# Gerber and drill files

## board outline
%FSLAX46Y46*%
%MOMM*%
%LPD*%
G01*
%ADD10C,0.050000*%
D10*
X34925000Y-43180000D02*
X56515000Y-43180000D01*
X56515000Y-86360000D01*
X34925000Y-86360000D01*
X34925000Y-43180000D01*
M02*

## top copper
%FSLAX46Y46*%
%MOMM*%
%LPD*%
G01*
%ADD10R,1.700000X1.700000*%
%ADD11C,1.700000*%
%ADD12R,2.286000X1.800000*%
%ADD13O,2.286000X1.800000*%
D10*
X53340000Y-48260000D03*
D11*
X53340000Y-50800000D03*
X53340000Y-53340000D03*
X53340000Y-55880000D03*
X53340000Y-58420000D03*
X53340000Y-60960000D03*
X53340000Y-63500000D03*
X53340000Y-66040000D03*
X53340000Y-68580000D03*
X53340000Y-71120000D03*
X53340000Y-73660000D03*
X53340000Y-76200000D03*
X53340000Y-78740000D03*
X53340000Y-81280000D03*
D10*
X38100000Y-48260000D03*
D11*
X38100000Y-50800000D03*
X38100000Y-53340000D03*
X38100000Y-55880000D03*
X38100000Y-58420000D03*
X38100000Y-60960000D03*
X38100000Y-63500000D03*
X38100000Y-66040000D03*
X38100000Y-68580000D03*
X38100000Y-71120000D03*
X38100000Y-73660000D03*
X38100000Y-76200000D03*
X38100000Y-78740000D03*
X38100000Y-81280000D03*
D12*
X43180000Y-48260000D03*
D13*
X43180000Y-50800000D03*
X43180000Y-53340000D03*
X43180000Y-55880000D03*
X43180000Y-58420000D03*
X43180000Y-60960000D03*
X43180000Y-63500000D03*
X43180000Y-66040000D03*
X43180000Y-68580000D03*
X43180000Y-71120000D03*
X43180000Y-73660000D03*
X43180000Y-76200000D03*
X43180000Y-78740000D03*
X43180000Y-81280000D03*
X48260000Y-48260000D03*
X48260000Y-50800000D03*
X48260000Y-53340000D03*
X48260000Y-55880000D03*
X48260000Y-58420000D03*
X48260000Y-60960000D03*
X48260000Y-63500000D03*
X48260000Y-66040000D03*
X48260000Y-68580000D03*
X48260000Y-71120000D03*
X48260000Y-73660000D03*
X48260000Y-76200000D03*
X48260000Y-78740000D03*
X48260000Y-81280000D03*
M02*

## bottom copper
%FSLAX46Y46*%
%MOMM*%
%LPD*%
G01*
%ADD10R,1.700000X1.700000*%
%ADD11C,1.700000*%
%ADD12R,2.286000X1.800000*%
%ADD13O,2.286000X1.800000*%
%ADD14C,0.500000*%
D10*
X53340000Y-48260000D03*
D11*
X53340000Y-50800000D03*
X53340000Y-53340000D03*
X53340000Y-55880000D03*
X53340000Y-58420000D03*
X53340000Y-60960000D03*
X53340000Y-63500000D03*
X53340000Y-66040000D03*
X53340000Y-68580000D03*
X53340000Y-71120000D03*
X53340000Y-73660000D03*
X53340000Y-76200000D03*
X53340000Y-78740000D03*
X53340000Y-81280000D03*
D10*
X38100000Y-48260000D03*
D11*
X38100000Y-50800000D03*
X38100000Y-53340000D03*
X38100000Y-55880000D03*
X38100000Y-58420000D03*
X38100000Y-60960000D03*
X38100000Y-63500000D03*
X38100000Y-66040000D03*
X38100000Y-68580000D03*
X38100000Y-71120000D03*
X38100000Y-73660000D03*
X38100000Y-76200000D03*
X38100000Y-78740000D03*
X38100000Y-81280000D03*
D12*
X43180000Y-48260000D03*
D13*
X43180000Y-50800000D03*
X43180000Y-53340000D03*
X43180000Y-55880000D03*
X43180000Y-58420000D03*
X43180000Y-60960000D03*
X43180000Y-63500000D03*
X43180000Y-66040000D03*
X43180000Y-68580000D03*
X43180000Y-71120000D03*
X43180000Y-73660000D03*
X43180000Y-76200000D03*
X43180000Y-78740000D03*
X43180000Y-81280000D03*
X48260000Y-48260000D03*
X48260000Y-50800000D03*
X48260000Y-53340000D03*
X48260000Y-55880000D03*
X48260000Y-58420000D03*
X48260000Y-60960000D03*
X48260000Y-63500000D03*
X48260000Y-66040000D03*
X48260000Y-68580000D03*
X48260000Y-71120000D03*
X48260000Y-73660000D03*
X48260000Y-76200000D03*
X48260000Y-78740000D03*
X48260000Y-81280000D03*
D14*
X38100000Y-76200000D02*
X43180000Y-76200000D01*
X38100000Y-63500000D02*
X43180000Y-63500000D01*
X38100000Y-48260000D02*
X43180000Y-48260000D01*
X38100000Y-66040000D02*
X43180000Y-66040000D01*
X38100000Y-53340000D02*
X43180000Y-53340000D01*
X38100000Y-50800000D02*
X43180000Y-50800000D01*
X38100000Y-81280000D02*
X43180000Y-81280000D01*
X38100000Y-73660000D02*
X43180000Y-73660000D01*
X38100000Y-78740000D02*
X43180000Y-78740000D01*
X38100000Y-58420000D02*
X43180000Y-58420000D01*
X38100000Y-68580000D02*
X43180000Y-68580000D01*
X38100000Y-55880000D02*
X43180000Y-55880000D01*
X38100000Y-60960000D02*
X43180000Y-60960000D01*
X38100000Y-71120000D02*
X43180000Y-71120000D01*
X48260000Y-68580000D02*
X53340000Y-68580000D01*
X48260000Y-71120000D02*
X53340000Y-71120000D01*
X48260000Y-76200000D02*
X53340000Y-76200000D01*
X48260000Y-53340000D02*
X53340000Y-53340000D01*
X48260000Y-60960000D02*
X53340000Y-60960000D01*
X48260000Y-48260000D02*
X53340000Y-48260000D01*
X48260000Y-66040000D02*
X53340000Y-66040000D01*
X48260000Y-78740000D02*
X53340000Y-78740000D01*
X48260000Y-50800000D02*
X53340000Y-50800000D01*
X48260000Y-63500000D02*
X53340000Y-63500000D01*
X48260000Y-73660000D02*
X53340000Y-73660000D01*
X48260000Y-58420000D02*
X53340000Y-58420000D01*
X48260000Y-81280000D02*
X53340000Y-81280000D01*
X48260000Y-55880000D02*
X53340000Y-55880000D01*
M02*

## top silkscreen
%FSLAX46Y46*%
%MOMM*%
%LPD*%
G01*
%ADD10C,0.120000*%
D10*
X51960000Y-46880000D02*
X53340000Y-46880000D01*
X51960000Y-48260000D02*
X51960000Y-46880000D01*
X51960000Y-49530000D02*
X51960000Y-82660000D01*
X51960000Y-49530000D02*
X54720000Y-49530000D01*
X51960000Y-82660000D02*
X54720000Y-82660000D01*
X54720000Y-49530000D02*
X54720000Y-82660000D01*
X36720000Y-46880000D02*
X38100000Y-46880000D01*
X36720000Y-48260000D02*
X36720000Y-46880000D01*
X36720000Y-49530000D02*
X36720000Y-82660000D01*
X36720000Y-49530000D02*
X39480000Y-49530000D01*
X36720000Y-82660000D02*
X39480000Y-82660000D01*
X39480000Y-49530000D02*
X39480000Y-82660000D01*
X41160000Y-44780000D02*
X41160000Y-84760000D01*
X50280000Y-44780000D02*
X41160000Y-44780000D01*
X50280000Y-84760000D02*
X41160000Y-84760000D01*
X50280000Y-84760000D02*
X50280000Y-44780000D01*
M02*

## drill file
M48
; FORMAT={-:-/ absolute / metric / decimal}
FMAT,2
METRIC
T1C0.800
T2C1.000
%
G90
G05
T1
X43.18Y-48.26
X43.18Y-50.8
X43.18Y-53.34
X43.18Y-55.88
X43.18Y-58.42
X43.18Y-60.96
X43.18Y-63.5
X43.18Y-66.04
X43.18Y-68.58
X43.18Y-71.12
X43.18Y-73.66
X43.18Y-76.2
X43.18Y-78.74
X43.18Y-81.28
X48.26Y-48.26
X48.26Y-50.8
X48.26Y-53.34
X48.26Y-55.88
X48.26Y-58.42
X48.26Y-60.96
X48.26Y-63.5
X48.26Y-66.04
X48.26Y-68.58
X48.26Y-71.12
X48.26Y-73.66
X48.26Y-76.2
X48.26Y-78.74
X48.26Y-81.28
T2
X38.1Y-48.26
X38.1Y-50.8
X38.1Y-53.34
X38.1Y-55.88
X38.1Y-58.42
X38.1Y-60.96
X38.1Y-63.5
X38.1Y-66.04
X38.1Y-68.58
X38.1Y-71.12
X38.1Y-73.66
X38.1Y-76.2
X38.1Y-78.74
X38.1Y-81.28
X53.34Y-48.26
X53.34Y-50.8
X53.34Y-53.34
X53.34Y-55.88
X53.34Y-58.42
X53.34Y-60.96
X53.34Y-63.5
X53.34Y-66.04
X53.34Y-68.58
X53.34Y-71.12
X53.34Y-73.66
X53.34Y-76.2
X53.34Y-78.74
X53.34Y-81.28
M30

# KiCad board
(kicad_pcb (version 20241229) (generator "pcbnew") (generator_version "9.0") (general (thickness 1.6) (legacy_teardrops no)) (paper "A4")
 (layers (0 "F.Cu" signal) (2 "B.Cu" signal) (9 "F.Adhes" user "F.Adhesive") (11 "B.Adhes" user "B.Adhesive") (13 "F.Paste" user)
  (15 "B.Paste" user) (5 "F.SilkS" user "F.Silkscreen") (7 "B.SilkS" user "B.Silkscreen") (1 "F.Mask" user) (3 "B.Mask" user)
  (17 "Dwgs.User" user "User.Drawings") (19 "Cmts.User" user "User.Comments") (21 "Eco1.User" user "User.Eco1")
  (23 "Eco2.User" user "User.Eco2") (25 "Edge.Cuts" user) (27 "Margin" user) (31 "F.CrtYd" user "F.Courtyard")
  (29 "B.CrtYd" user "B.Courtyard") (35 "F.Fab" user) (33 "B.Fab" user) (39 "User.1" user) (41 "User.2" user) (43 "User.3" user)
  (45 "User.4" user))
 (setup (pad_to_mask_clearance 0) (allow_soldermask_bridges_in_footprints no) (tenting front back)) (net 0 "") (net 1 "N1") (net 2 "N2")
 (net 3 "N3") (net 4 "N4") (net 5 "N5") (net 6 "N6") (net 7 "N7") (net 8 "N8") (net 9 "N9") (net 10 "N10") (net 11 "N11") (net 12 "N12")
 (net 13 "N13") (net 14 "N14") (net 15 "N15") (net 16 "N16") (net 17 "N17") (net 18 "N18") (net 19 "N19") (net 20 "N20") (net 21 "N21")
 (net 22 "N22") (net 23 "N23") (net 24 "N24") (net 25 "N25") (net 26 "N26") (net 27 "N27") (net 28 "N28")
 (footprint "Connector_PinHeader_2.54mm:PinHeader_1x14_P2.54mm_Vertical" (layer "F.Cu") (at 53.34 48.26)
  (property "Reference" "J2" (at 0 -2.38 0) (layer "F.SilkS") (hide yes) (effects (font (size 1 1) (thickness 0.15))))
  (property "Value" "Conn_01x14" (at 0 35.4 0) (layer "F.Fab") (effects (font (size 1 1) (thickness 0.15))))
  (fp_line (start -1.38 -1.38) (end 0 -1.38) (stroke (width 0.12) (type solid)) (layer "F.SilkS"))
  (fp_line (start -1.38 0) (end -1.38 -1.38) (stroke (width 0.12) (type solid)) (layer "F.SilkS"))
  (fp_line (start -1.38 1.27) (end -1.38 34.4) (stroke (width 0.12) (type solid)) (layer "F.SilkS"))
  (fp_line (start -1.38 1.27) (end 1.38 1.27) (stroke (width 0.12) (type solid)) (layer "F.SilkS"))
  (fp_line (start -1.38 34.4) (end 1.38 34.4) (stroke (width 0.12) (type solid)) (layer "F.SilkS"))
  (fp_line (start 1.38 1.27) (end 1.38 34.4) (stroke (width 0.12) (type solid)) (layer "F.SilkS"))
  (pad "1" thru_hole rect (at 0 0) (size 1.7 1.7) (drill 1) (layers "*.Cu" "*.Mask") (remove_unused_layers no) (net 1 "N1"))
  (pad "2" thru_hole circle (at 0 2.54) (size 1.7 1.7) (drill 1) (layers "*.Cu" "*.Mask") (remove_unused_layers no) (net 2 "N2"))
  (pad "3" thru_hole circle (at 0 5.08) (size 1.7 1.7) (drill 1) (layers "*.Cu" "*.Mask") (remove_unused_layers no) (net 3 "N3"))
  (pad "4" thru_hole circle (at 0 7.62) (size 1.7 1.7) (drill 1) (layers "*.Cu" "*.Mask") (remove_unused_layers no) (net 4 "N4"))
  (pad "5" thru_hole circle (at 0 10.16) (size 1.7 1.7) (drill 1) (layers "*.Cu" "*.Mask") (remove_unused_layers no) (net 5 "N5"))
  (pad "6" thru_hole circle (at 0 12.7) (size 1.7 1.7) (drill 1) (layers "*.Cu" "*.Mask") (remove_unused_layers no) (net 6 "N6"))
  (pad "7" thru_hole circle (at 0 15.24) (size 1.7 1.7) (drill 1) (layers "*.Cu" "*.Mask") (remove_unused_layers no) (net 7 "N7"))
  (pad "8" thru_hole circle (at 0 17.78) (size 1.7 1.7) (drill 1) (layers "*.Cu" "*.Mask") (remove_unused_layers no) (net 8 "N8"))
  (pad "9" thru_hole circle (at 0 20.32) (size 1.7 1.7) (drill 1) (layers "*.Cu" "*.Mask") (remove_unused_layers no) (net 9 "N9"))
  (pad "10" thru_hole circle (at 0 22.86) (size 1.7 1.7) (drill 1) (layers "*.Cu" "*.Mask") (remove_unused_layers no) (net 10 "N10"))
  (pad "11" thru_hole circle (at 0 25.4) (size 1.7 1.7) (drill 1) (layers "*.Cu" "*.Mask") (remove_unused_layers no) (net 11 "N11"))
  (pad "12" thru_hole circle (at 0 27.94) (size 1.7 1.7) (drill 1) (layers "*.Cu" "*.Mask") (remove_unused_layers no) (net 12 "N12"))
  (pad "13" thru_hole circle (at 0 30.48) (size 1.7 1.7) (drill 1) (layers "*.Cu" "*.Mask") (remove_unused_layers no) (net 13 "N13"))
  (pad "14" thru_hole circle (at 0 33.02) (size 1.7 1.7) (drill 1) (layers "*.Cu" "*.Mask") (remove_unused_layers no) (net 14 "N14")))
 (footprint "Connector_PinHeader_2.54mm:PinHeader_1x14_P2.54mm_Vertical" (layer "F.Cu") (at 38.1 48.26)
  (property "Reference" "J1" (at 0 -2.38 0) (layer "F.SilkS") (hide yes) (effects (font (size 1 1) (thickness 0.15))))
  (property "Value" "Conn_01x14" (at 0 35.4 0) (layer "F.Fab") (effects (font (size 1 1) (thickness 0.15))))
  (fp_line (start -1.38 -1.38) (end 0 -1.38) (stroke (width 0.12) (type solid)) (layer "F.SilkS"))
  (fp_line (start -1.38 0) (end -1.38 -1.38) (stroke (width 0.12) (type solid)) (layer "F.SilkS"))
  (fp_line (start -1.38 1.27) (end -1.38 34.4) (stroke (width 0.12) (type solid)) (layer "F.SilkS"))
  (fp_line (start -1.38 1.27) (end 1.38 1.27) (stroke (width 0.12) (type solid)) (layer "F.SilkS"))
  (fp_line (start -1.38 34.4) (end 1.38 34.4) (stroke (width 0.12) (type solid)) (layer "F.SilkS"))
  (fp_line (start 1.38 1.27) (end 1.38 34.4) (stroke (width 0.12) (type solid)) (layer "F.SilkS"))
  (pad "1" thru_hole rect (at 0 0) (size 1.7 1.7) (drill 1) (layers "*.Cu" "*.Mask") (remove_unused_layers no) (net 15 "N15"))
  (pad "2" thru_hole circle (at 0 2.54) (size 1.7 1.7) (drill 1) (layers "*.Cu" "*.Mask") (remove_unused_layers no) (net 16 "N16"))
  (pad "3" thru_hole circle (at 0 5.08) (size 1.7 1.7) (drill 1) (layers "*.Cu" "*.Mask") (remove_unused_layers no) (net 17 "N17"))
  (pad "4" thru_hole circle (at 0 7.62) (size 1.7 1.7) (drill 1) (layers "*.Cu" "*.Mask") (remove_unused_layers no) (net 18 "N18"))
  (pad "5" thru_hole circle (at 0 10.16) (size 1.7 1.7) (drill 1) (layers "*.Cu" "*.Mask") (remove_unused_layers no) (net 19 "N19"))
  (pad "6" thru_hole circle (at 0 12.7) (size 1.7 1.7) (drill 1) (layers "*.Cu" "*.Mask") (remove_unused_layers no) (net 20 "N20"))
  (pad "7" thru_hole circle (at 0 15.24) (size 1.7 1.7) (drill 1) (layers "*.Cu" "*.Mask") (remove_unused_layers no) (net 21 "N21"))
  (pad "8" thru_hole circle (at 0 17.78) (size 1.7 1.7) (drill 1) (layers "*.Cu" "*.Mask") (remove_unused_layers no) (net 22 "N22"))
  (pad "9" thru_hole circle (at 0 20.32) (size 1.7 1.7) (drill 1) (layers "*.Cu" "*.Mask") (remove_unused_layers no) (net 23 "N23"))
  (pad "10" thru_hole circle (at 0 22.86) (size 1.7 1.7) (drill 1) (layers "*.Cu" "*.Mask") (remove_unused_layers no) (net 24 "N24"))
  (pad "11" thru_hole circle (at 0 25.4) (size 1.7 1.7) (drill 1) (layers "*.Cu" "*.Mask") (remove_unused_layers no) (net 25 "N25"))
  (pad "12" thru_hole circle (at 0 27.94) (size 1.7 1.7) (drill 1) (layers "*.Cu" "*.Mask") (remove_unused_layers no) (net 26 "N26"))
  (pad "13" thru_hole circle (at 0 30.48) (size 1.7 1.7) (drill 1) (layers "*.Cu" "*.Mask") (remove_unused_layers no) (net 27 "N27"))
  (pad "14" thru_hole circle (at 0 33.02) (size 1.7 1.7) (drill 1) (layers "*.Cu" "*.Mask") (remove_unused_layers no) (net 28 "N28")))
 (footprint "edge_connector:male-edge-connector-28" (layer "F.Cu") (at 43.18 48.26)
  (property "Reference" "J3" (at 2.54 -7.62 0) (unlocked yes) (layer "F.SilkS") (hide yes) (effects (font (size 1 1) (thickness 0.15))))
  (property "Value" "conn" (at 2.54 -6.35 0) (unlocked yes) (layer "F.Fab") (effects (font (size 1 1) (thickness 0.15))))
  (fp_line (start -2.02 -3.48) (end -2.02 36.5) (stroke (width 0.12) (type solid)) (layer "F.SilkS"))
  (fp_line (start 7.1 -3.48) (end -2.02 -3.48) (stroke (width 0.12) (type solid)) (layer "F.SilkS"))
  (fp_line (start 7.1 36.5) (end -2.02 36.5) (stroke (width 0.12) (type solid)) (layer "F.SilkS"))
  (fp_line (start 7.1 36.5) (end 7.1 -3.48) (stroke (width 0.12) (type solid)) (layer "F.SilkS"))
  (pad "1" thru_hole rect (at 0 0) (size 2.286 1.8) (drill 0.8) (layers "*.Cu" "*.Mask") (remove_unused_layers yes) (keep_end_layers yes)
   (zone_layer_connections) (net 15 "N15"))
  (pad "2" thru_hole oval (at 0 2.54) (size 2.286 1.8) (drill 0.8) (layers "*.Cu" "*.Mask") (remove_unused_layers no) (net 16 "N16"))
  (pad "3" thru_hole oval (at 0 5.08) (size 2.286 1.8) (drill 0.8) (layers "*.Cu" "*.Mask") (remove_unused_layers no) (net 17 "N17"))
  (pad "4" thru_hole oval (at 0 7.62) (size 2.286 1.8) (drill 0.8) (layers "*.Cu" "*.Mask") (remove_unused_layers no) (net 18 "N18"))
  (pad "5" thru_hole oval (at 0 10.16) (size 2.286 1.8) (drill 0.8) (layers "*.Cu" "*.Mask") (remove_unused_layers no) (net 19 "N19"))
  (pad "6" thru_hole oval (at 0 12.7) (size 2.286 1.8) (drill 0.8) (layers "*.Cu" "*.Mask") (remove_unused_layers no) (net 20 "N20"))
  (pad "7" thru_hole oval (at 0 15.24) (size 2.286 1.8) (drill 0.8) (layers "*.Cu" "*.Mask") (remove_unused_layers no) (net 21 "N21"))
  (pad "8" thru_hole oval (at 0 17.78) (size 2.286 1.8) (drill 0.8) (layers "*.Cu" "*.Mask") (remove_unused_layers no) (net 22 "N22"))
  (pad "9" thru_hole oval (at 0 20.32) (size 2.286 1.8) (drill 0.8) (layers "*.Cu" "*.Mask") (remove_unused_layers no) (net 23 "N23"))
  (pad "10" thru_hole oval (at 0 22.86) (size 2.286 1.8) (drill 0.8) (layers "*.Cu" "*.Mask") (remove_unused_layers no) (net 24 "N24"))
  (pad "11" thru_hole oval (at 0 25.4) (size 2.286 1.8) (drill 0.8) (layers "*.Cu" "*.Mask") (remove_unused_layers no) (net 25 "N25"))
  (pad "12" thru_hole oval (at 0 27.94) (size 2.286 1.8) (drill 0.8) (layers "*.Cu" "*.Mask") (remove_unused_layers no) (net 26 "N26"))
  (pad "13" thru_hole oval (at 0 30.48) (size 2.286 1.8) (drill 0.8) (layers "*.Cu" "*.Mask") (remove_unused_layers no) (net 27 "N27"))
  (pad "14" thru_hole oval (at 0 33.02) (size 2.286 1.8) (drill 0.8) (layers "*.Cu" "*.Mask") (remove_unused_layers no) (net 28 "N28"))
  (pad "15" thru_hole oval (at 5.08 0) (size 2.286 1.8) (drill 0.8) (layers "*.Cu" "*.Mask") (remove_unused_layers no) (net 1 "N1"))
  (pad "16" thru_hole oval (at 5.08 2.54) (size 2.286 1.8) (drill 0.8) (layers "*.Cu" "*.Mask") (remove_unused_layers no) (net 2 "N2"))
  (pad "17" thru_hole oval (at 5.08 5.08) (size 2.286 1.8) (drill 0.8) (layers "*.Cu" "*.Mask") (remove_unused_layers no) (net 3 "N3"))
  (pad "18" thru_hole oval (at 5.08 7.62) (size 2.286 1.8) (drill 0.8) (layers "*.Cu" "*.Mask") (remove_unused_layers no) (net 4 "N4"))
  (pad "19" thru_hole oval (at 5.08 10.16) (size 2.286 1.8) (drill 0.8) (layers "*.Cu" "*.Mask") (remove_unused_layers no) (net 5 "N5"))
  (pad "20" thru_hole oval (at 5.08 12.7) (size 2.286 1.8) (drill 0.8) (layers "*.Cu" "*.Mask") (remove_unused_layers no) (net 6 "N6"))
  (pad "21" thru_hole oval (at 5.08 15.24) (size 2.286 1.8) (drill 0.8) (layers "*.Cu" "*.Mask") (remove_unused_layers no) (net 7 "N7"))
  (pad "22" thru_hole oval (at 5.08 17.78) (size 2.286 1.8) (drill 0.8) (layers "*.Cu" "*.Mask") (remove_unused_layers no) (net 8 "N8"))
  (pad "23" thru_hole oval (at 5.08 20.32) (size 2.286 1.8) (drill 0.8) (layers "*.Cu" "*.Mask") (remove_unused_layers no) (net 9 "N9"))
  (pad "24" thru_hole oval (at 5.08 22.86) (size 2.286 1.8) (drill 0.8) (layers "*.Cu" "*.Mask") (remove_unused_layers no) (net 10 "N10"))
  (pad "25" thru_hole oval (at 5.08 25.4) (size 2.286 1.8) (drill 0.8) (layers "*.Cu" "*.Mask") (remove_unused_layers no) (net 11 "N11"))
  (pad "26" thru_hole oval (at 5.08 27.94) (size 2.286 1.8) (drill 0.8) (layers "*.Cu" "*.Mask") (remove_unused_layers no) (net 12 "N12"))
  (pad "27" thru_hole oval (at 5.08 30.48) (size 2.286 1.8) (drill 0.8) (layers "*.Cu" "*.Mask") (remove_unused_layers no) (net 13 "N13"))
  (pad "28" thru_hole oval (at 5.08 33.02) (size 2.286 1.8) (drill 0.8) (layers "*.Cu" "*.Mask") (remove_unused_layers no) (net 14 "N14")))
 (gr_rect (start 34.925 43.18) (end 56.515 86.36) (stroke (width 0.05) (type default)) (fill no) (layer "Edge.Cuts"))
 (segment (start 38.1 76.2) (end 43.18 76.2) (width 0.5) (layer "B.Cu") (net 26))
 (segment (start 38.1 63.5) (end 43.18 63.5) (width 0.5) (layer "B.Cu") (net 21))
 (segment (start 38.1 48.26) (end 43.18 48.26) (width 0.5) (layer "B.Cu") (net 15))
 (segment (start 38.1 66.04) (end 43.18 66.04) (width 0.5) (layer "B.Cu") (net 22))
 (segment (start 38.1 53.34) (end 43.18 53.34) (width 0.5) (layer "B.Cu") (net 17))
 (segment (start 38.1 50.8) (end 43.18 50.8) (width 0.5) (layer "B.Cu") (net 16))
 (segment (start 38.1 81.28) (end 43.18 81.28) (width 0.5) (layer "B.Cu") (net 28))
 (segment (start 38.1 73.66) (end 43.18 73.66) (width 0.5) (layer "B.Cu") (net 25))
 (segment (start 38.1 78.74) (end 43.18 78.74) (width 0.5) (layer "B.Cu") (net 27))
 (segment (start 38.1 58.42) (end 43.18 58.42) (width 0.5) (layer "B.Cu") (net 19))
 (segment (start 38.1 68.58) (end 43.18 68.58) (width 0.5) (layer "B.Cu") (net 23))
 (segment (start 38.1 55.88) (end 43.18 55.88) (width 0.5) (layer "B.Cu") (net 18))
 (segment (start 38.1 60.96) (end 43.18 60.96) (width 0.5) (layer "B.Cu") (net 20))
 (segment (start 38.1 71.12) (end 43.18 71.12) (width 0.5) (layer "B.Cu") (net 24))
 (segment (start 48.26 68.58) (end 53.34 68.58) (width 0.5) (layer "B.Cu") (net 9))
 (segment (start 48.26 71.12) (end 53.34 71.12) (width 0.5) (layer "B.Cu") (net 10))
 (segment (start 48.26 76.2) (end 53.34 76.2) (width 0.5) (layer "B.Cu") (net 12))
 (segment (start 48.26 53.34) (end 53.34 53.34) (width 0.5) (layer "B.Cu") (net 3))
 (segment (start 48.26 60.96) (end 53.34 60.96) (width 0.5) (layer "B.Cu") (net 6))
 (segment (start 48.26 48.26) (end 53.34 48.26) (width 0.5) (layer "B.Cu") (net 1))
 (segment (start 48.26 66.04) (end 53.34 66.04) (width 0.5) (layer "B.Cu") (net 8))
 (segment (start 48.26 78.74) (end 53.34 78.74) (width 0.5) (layer "B.Cu") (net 13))
 (segment (start 48.26 50.8) (end 53.34 50.8) (width 0.5) (layer "B.Cu") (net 2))
 (segment (start 48.26 63.5) (end 53.34 63.5) (width 0.5) (layer "B.Cu") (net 7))
 (segment (start 48.26 73.66) (end 53.34 73.66) (width 0.5) (layer "B.Cu") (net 11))
 (segment (start 48.26 58.42) (end 53.34 58.42) (width 0.5) (layer "B.Cu") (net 5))
 (segment (start 48.26 81.28) (end 53.34 81.28) (width 0.5) (layer "B.Cu") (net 14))
 (segment (start 48.26 55.88) (end 53.34 55.88) (width 0.5) (layer "B.Cu") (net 4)))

